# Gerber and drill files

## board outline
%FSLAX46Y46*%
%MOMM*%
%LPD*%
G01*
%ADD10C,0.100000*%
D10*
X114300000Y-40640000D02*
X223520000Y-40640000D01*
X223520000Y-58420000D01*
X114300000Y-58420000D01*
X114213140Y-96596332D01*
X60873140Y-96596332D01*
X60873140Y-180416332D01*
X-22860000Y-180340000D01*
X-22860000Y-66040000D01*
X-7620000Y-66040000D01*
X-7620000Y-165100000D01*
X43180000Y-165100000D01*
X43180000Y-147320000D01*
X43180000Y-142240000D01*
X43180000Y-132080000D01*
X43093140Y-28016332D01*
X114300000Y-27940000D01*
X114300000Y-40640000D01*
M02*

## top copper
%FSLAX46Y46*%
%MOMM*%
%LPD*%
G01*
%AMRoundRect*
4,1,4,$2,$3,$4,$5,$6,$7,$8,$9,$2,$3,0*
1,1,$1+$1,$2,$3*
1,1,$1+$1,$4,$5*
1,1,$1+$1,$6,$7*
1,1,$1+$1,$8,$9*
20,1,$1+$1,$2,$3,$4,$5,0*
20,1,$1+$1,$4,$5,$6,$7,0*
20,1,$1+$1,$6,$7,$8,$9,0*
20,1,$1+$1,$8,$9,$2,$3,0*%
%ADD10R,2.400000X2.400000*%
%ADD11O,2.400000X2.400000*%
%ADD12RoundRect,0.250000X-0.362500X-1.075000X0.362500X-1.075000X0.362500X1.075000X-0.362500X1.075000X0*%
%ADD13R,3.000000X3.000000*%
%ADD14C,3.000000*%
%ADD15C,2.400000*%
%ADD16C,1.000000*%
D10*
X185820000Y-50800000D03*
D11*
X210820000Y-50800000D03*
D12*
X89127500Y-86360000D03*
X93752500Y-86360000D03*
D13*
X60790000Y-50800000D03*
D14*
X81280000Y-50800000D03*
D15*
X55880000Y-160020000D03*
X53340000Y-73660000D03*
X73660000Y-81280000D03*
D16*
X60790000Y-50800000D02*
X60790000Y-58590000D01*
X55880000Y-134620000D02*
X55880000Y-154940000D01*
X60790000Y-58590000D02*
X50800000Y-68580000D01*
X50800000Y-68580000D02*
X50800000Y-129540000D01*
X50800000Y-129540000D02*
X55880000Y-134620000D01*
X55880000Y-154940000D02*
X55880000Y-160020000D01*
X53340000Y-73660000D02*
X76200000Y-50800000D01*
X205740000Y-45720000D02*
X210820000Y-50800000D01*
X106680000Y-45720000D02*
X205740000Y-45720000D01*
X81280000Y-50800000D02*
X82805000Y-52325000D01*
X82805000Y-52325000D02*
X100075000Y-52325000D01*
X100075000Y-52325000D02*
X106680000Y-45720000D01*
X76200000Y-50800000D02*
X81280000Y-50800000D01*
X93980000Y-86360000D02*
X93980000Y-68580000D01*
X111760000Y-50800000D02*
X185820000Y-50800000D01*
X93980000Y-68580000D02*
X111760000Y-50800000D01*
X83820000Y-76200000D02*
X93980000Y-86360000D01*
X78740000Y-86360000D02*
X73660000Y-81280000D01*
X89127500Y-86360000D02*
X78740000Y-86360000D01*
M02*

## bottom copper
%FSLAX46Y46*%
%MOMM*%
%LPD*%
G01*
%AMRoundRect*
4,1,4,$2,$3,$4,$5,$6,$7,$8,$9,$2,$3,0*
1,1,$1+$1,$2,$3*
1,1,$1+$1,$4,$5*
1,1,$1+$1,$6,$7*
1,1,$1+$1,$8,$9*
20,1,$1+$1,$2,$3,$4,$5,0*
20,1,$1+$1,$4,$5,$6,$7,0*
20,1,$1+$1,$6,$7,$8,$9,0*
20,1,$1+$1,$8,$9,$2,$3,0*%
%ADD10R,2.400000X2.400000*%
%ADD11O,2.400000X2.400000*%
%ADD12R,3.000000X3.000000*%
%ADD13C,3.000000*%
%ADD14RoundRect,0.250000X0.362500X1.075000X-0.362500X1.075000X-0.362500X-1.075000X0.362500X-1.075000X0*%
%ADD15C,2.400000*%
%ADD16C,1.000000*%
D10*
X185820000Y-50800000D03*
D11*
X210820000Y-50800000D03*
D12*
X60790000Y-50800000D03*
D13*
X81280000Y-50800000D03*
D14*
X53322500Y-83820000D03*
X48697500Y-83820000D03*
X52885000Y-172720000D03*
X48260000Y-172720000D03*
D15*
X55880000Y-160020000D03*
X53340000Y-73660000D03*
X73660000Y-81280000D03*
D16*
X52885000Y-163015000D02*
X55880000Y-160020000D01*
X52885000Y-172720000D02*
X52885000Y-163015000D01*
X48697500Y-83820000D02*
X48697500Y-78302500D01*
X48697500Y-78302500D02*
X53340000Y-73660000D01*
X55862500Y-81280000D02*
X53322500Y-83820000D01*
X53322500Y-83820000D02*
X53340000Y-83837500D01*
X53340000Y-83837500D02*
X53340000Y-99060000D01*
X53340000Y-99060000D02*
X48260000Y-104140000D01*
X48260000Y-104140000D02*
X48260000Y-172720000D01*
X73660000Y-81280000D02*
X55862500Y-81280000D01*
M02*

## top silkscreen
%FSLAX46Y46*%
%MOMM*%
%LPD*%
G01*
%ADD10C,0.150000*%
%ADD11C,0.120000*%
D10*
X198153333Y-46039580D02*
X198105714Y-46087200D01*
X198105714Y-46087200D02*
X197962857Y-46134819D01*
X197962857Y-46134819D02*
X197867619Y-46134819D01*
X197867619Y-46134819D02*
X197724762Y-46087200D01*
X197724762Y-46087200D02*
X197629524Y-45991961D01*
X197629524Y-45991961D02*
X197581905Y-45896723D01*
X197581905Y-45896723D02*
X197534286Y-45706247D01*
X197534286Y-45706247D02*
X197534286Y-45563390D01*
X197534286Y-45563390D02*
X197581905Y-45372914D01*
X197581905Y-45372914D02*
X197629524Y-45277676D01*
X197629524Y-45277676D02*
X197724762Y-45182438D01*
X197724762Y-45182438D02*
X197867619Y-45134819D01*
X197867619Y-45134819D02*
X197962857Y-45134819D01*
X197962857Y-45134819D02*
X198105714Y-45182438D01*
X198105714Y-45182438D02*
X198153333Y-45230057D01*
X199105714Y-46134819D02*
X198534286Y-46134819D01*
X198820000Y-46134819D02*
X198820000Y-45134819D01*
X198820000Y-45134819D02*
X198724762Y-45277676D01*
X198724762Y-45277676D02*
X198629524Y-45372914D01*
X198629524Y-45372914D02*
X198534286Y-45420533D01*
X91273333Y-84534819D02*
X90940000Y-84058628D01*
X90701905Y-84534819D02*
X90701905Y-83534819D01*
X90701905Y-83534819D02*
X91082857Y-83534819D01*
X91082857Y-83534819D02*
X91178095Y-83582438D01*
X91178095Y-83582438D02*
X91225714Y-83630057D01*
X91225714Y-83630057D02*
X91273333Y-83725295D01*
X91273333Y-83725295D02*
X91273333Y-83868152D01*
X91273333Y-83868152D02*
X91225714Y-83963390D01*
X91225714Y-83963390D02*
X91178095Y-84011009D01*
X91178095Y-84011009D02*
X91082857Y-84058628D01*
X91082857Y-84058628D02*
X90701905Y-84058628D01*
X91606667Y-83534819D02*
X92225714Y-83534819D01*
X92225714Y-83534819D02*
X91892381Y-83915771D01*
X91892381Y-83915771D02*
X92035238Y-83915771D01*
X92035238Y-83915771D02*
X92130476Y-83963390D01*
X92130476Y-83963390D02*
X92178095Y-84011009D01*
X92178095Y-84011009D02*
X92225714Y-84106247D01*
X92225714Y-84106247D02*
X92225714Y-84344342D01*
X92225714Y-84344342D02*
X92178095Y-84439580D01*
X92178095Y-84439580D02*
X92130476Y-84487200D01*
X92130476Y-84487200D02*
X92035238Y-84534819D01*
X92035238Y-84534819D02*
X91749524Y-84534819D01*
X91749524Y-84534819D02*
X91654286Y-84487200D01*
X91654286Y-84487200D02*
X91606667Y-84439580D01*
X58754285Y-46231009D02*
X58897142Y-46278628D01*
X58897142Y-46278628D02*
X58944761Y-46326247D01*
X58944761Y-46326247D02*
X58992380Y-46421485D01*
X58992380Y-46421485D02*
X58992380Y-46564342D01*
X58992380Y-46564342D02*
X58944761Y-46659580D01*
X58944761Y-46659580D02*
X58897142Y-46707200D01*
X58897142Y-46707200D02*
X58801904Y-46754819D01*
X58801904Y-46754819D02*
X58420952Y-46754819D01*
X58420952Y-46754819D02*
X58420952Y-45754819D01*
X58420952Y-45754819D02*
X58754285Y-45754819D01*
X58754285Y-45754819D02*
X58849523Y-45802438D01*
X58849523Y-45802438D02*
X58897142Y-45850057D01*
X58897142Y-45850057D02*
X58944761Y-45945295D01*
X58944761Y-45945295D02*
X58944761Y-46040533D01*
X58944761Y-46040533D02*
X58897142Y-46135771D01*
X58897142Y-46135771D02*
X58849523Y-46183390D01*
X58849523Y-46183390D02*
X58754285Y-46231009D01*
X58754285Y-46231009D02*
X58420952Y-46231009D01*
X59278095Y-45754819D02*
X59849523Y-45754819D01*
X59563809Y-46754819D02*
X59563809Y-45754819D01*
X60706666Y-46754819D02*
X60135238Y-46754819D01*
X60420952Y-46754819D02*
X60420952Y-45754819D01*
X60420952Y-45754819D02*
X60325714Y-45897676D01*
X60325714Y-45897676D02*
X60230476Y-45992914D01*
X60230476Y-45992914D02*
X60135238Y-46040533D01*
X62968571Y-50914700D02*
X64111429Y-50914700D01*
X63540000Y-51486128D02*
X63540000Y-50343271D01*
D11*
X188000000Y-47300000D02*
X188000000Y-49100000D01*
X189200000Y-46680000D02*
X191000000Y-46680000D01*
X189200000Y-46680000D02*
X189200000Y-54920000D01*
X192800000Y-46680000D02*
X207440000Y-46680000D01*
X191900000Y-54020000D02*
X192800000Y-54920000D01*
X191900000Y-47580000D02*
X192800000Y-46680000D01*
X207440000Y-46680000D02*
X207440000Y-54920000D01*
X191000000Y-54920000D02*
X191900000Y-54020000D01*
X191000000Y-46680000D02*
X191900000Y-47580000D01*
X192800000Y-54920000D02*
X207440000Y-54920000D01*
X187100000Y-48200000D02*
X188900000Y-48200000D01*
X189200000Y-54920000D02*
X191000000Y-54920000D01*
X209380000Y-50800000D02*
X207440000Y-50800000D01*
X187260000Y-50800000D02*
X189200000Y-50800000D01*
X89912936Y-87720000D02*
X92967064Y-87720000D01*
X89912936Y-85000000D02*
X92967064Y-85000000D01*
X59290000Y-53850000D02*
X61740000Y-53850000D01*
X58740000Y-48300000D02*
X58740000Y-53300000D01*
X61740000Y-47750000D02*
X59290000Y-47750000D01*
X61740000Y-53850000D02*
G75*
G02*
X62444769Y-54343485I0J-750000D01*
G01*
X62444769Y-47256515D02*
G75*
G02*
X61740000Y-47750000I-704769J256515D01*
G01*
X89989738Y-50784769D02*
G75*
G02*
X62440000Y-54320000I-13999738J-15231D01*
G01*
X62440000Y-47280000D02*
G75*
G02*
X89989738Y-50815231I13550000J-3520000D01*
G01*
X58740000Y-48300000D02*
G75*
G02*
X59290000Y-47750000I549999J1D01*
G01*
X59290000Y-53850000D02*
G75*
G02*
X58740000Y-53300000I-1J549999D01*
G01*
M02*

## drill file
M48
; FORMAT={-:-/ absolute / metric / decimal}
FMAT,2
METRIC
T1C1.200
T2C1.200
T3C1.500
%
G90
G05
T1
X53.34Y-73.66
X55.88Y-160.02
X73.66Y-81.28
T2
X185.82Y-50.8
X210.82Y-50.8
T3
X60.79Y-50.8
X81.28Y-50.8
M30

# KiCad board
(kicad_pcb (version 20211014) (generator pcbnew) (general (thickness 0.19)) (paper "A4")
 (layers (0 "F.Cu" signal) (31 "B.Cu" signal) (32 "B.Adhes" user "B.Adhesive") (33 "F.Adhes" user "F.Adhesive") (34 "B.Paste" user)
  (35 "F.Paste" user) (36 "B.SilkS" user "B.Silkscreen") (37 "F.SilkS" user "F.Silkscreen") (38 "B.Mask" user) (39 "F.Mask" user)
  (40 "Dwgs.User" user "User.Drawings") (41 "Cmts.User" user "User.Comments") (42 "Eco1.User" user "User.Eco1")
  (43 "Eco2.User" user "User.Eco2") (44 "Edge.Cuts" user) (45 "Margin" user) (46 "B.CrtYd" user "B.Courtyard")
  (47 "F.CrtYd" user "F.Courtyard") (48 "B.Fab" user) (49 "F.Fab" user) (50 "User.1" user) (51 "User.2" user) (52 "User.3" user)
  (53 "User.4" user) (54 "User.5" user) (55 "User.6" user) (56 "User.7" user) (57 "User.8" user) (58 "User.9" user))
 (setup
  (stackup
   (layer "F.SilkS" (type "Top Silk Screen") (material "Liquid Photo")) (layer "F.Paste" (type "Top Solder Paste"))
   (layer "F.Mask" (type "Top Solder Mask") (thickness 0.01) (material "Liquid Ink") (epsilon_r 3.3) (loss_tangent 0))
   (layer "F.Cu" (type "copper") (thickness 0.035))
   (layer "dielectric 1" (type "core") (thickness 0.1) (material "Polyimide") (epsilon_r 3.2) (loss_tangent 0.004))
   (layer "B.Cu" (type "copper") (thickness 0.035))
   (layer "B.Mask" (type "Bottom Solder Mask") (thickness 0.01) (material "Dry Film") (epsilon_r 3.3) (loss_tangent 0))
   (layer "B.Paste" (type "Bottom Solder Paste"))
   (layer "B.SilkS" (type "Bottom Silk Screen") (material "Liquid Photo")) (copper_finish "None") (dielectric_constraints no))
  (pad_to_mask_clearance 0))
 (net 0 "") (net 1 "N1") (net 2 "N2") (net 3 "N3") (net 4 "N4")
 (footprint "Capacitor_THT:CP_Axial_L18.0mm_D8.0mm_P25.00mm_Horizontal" (layer "F.Cu") (at 185.82 50.8)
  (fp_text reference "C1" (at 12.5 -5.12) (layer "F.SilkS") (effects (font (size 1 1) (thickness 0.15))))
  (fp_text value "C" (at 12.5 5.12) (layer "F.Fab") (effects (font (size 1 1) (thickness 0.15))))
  (fp_line (start 2.18 -3.5) (end 2.18 -1.7) (layer "F.SilkS") (width 0.12))
  (fp_line (start 3.38 -4.12) (end 5.18 -4.12) (layer "F.SilkS") (width 0.12))
  (fp_line (start 3.38 -4.12) (end 3.38 4.12) (layer "F.SilkS") (width 0.12))
  (fp_line (start 6.98 -4.12) (end 21.62 -4.12) (layer "F.SilkS") (width 0.12))
  (fp_line (start 6.08 3.22) (end 6.98 4.12) (layer "F.SilkS") (width 0.12))
  (fp_line (start 6.08 -3.22) (end 6.98 -4.12) (layer "F.SilkS") (width 0.12))
  (fp_line (start 21.62 -4.12) (end 21.62 4.12) (layer "F.SilkS") (width 0.12))
  (fp_line (start 5.18 4.12) (end 6.08 3.22) (layer "F.SilkS") (width 0.12))
  (fp_line (start 5.18 -4.12) (end 6.08 -3.22) (layer "F.SilkS") (width 0.12))
  (fp_line (start 6.98 4.12) (end 21.62 4.12) (layer "F.SilkS") (width 0.12))
  (fp_line (start 1.28 -2.6) (end 3.08 -2.6) (layer "F.SilkS") (width 0.12))
  (fp_line (start 3.38 4.12) (end 5.18 4.12) (layer "F.SilkS") (width 0.12))
  (fp_line (start 23.56 0) (end 21.62 0) (layer "F.SilkS") (width 0.12))
  (fp_line (start 1.44 0) (end 3.38 0) (layer "F.SilkS") (width 0.12))
  (pad "1" thru_hole rect (at 0 0) (size 2.4 2.4) (drill 1.2) (layers *.Cu *.Mask) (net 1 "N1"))
  (pad "2" thru_hole oval (at 25 0) (size 2.4 2.4) (drill 1.2) (layers *.Cu *.Mask) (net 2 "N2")))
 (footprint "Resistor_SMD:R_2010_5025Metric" (layer "F.Cu") (at 91.44 86.36)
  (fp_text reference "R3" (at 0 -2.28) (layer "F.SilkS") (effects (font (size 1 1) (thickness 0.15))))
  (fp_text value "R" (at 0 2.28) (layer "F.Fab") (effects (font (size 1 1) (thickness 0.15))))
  (fp_line (start -1.527064 1.36) (end 1.527064 1.36) (layer "F.SilkS") (width 0.12))
  (fp_line (start -1.527064 -1.36) (end 1.527064 -1.36) (layer "F.SilkS") (width 0.12))
  (pad "1" smd roundrect (at -2.3125 0) (size 1.225 2.65) (layers "F.Cu" "F.Paste" "F.Mask") (roundrect_rratio 0.204082) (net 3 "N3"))
  (pad "2" smd roundrect (at 2.3125 0) (size 1.225 2.65) (layers "F.Cu" "F.Paste" "F.Mask") (roundrect_rratio 0.204082) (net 1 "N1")))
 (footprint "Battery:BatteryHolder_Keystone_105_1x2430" (layer "F.Cu") (at 60.79 50.8)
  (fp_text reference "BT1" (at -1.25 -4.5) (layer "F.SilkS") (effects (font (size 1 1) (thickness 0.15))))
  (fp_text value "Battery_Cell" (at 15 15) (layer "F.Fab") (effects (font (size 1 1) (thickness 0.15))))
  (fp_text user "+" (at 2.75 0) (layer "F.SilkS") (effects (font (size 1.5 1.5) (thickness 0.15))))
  (fp_line (start -1.5 3.05) (end 0.95 3.05) (layer "F.SilkS") (width 0.12))
  (fp_line (start -2.05 -2.5) (end -2.05 2.5) (layer "F.SilkS") (width 0.12))
  (fp_line (start 0.95 -3.05) (end -1.5 -3.05) (layer "F.SilkS") (width 0.12))
  (fp_arc (start 0.95 3.05) (mid 1.380182 3.185636) (end 1.654769 3.543485) (layer "F.SilkS") (width 0.12))
  (fp_arc (start 1.654769 -3.543485) (mid 1.380182 -3.185636) (end 0.95 -3.05) (layer "F.SilkS") (width 0.12))
  (fp_arc (start 29.199738 -0.015231) (mid 16.981862 13.885887) (end 1.65 3.52) (layer "F.SilkS") (width 0.12))
  (fp_arc (start 1.65 -3.52) (mid 16.981862 -13.885887) (end 29.199738 0.015231) (layer "F.SilkS") (width 0.12))
  (fp_arc (start -2.05 -2.5) (mid -1.888909 -2.888909) (end -1.5 -3.05) (layer "F.SilkS") (width 0.12))
  (fp_arc (start -1.5 3.05) (mid -1.888909 2.888909) (end -2.05 2.5) (layer "F.SilkS") (width 0.12))
  (pad "1" thru_hole rect (at 0 0) (size 3 3) (drill 1.5) (layers *.Cu *.Mask) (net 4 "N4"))
  (pad "2" thru_hole circle (at 20.49 0) (size 3 3) (drill 1.5) (layers *.Cu *.Mask) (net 2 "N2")))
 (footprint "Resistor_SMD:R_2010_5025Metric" (layer "B.Cu") (at 51.01 83.82 180)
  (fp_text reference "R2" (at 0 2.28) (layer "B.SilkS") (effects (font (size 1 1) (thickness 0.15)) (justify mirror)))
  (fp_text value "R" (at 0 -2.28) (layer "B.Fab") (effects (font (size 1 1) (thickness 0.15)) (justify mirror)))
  (pad "1" smd roundrect (at -2.3125 0 180) (size 1.225 2.65) (layers "B.Cu" "B.Paste" "B.Mask") (roundrect_rratio 0.204082) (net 3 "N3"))
  (pad "2" smd roundrect (at 2.3125 0 180) (size 1.225 2.65) (layers "B.Cu" "B.Paste" "B.Mask") (roundrect_rratio 0.204082) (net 2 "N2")))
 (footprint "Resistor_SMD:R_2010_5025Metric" (layer "B.Cu") (at 50.5725 172.72 180)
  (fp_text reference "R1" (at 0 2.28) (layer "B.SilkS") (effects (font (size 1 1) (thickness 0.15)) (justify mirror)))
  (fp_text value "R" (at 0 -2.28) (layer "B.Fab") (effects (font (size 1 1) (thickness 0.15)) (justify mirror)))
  (pad "1" smd roundrect (at -2.3125 0 180) (size 1.225 2.65) (layers "B.Cu" "B.Paste" "B.Mask") (roundrect_rratio 0.204082) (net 4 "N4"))
  (pad "2" smd roundrect (at 2.3125 0 180) (size 1.225 2.65) (layers "B.Cu" "B.Paste" "B.Mask") (roundrect_rratio 0.204082) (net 3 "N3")))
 (gr_poly
  (pts (xy 114.3 40.64) (xy 223.52 40.64) (xy 223.52 58.42) (xy 114.3 58.42) (xy 114.21314 96.596332) (xy 60.87314 96.596332)
   (xy 60.87314 180.416332) (xy -22.86 180.34) (xy -22.86 66.04) (xy -7.62 66.04) (xy -7.62 165.1) (xy 43.18 165.1) (xy 43.18 147.32)
   (xy 43.18 142.24) (xy 43.18 132.08) (xy 43.09314 28.016332) (xy 114.3 27.94))
  (layer "Edge.Cuts") (width 0.1) (fill none))
 (segment (start 60.79 50.8) (end 60.79 58.59) (width 1) (layer "F.Cu") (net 4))
 (segment (start 55.88 134.62) (end 55.88 154.94) (width 1) (layer "F.Cu") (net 4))
 (segment (start 60.79 58.59) (end 50.8 68.58) (width 1) (layer "F.Cu") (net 4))
 (segment (start 50.8 68.58) (end 50.8 129.54) (width 1) (layer "F.Cu") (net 4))
 (segment (start 50.8 129.54) (end 55.88 134.62) (width 1) (layer "F.Cu") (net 4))
 (segment (start 55.88 154.94) (end 55.88 160.02) (width 1) (layer "F.Cu") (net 4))
 (via (at 55.88 160.02) (size 2.4) (drill 1.2) (layers "F.Cu" "B.Cu") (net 4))
 (segment (start 52.885 163.015) (end 55.88 160.02) (width 1) (layer "B.Cu") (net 4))
 (segment (start 52.885 172.72) (end 52.885 163.015) (width 1) (layer "B.Cu") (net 4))
 (segment (start 53.34 73.66) (end 76.2 50.8) (width 1) (layer "F.Cu") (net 2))
 (segment (start 205.74 45.72) (end 210.82 50.8) (width 1) (layer "F.Cu") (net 2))
 (segment (start 106.68 45.72) (end 205.74 45.72) (width 1) (layer "F.Cu") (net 2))
 (segment (start 81.28 50.8) (end 82.805 52.325) (width 1) (layer "F.Cu") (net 2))
 (segment (start 82.805 52.325) (end 100.075 52.325) (width 1) (layer "F.Cu") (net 2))
 (segment (start 100.075 52.325) (end 106.68 45.72) (width 1) (layer "F.Cu") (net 2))
 (segment (start 76.2 50.8) (end 81.28 50.8) (width 1) (layer "F.Cu") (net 2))
 (via (at 53.34 73.66) (size 2.4) (drill 1.2) (layers "F.Cu" "B.Cu") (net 2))
 (segment (start 48.6975 83.82) (end 48.6975 78.3025) (width 1) (layer "B.Cu") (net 2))
 (segment (start 48.6975 78.3025) (end 53.34 73.66) (width 1) (layer "B.Cu") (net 2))
 (segment (start 93.98 86.36) (end 93.98 68.58) (width 1) (layer "F.Cu") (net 1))
 (segment (start 111.76 50.8) (end 185.82 50.8) (width 1) (layer "F.Cu") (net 1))
 (segment (start 93.98 68.58) (end 111.76 50.8) (width 1) (layer "F.Cu") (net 1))
 (segment (start 83.82 76.2) (end 93.98 86.36) (width 1) (layer "F.Cu") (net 1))
 (segment (start 78.74 86.36) (end 73.66 81.28) (width 1) (layer "F.Cu") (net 3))
 (segment (start 89.1275 86.36) (end 78.74 86.36) (width 1) (layer "F.Cu") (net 3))
 (via (at 73.66 81.28) (size 2.4) (drill 1.2) (layers "F.Cu" "B.Cu") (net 3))
 (segment (start 55.8625 81.28) (end 53.3225 83.82) (width 1) (layer "B.Cu") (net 3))
 (segment (start 53.3225 83.82) (end 53.34 83.8375) (width 1) (layer "B.Cu") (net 3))
 (segment (start 53.34 83.8375) (end 53.34 99.06) (width 1) (layer "B.Cu") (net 3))
 (segment (start 53.34 99.06) (end 48.26 104.14) (width 1) (layer "B.Cu") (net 3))
 (segment (start 48.26 104.14) (end 48.26 172.72) (width 1) (layer "B.Cu") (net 3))
 (segment (start 73.66 81.28) (end 55.8625 81.28) (width 1) (layer "B.Cu") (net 3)))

